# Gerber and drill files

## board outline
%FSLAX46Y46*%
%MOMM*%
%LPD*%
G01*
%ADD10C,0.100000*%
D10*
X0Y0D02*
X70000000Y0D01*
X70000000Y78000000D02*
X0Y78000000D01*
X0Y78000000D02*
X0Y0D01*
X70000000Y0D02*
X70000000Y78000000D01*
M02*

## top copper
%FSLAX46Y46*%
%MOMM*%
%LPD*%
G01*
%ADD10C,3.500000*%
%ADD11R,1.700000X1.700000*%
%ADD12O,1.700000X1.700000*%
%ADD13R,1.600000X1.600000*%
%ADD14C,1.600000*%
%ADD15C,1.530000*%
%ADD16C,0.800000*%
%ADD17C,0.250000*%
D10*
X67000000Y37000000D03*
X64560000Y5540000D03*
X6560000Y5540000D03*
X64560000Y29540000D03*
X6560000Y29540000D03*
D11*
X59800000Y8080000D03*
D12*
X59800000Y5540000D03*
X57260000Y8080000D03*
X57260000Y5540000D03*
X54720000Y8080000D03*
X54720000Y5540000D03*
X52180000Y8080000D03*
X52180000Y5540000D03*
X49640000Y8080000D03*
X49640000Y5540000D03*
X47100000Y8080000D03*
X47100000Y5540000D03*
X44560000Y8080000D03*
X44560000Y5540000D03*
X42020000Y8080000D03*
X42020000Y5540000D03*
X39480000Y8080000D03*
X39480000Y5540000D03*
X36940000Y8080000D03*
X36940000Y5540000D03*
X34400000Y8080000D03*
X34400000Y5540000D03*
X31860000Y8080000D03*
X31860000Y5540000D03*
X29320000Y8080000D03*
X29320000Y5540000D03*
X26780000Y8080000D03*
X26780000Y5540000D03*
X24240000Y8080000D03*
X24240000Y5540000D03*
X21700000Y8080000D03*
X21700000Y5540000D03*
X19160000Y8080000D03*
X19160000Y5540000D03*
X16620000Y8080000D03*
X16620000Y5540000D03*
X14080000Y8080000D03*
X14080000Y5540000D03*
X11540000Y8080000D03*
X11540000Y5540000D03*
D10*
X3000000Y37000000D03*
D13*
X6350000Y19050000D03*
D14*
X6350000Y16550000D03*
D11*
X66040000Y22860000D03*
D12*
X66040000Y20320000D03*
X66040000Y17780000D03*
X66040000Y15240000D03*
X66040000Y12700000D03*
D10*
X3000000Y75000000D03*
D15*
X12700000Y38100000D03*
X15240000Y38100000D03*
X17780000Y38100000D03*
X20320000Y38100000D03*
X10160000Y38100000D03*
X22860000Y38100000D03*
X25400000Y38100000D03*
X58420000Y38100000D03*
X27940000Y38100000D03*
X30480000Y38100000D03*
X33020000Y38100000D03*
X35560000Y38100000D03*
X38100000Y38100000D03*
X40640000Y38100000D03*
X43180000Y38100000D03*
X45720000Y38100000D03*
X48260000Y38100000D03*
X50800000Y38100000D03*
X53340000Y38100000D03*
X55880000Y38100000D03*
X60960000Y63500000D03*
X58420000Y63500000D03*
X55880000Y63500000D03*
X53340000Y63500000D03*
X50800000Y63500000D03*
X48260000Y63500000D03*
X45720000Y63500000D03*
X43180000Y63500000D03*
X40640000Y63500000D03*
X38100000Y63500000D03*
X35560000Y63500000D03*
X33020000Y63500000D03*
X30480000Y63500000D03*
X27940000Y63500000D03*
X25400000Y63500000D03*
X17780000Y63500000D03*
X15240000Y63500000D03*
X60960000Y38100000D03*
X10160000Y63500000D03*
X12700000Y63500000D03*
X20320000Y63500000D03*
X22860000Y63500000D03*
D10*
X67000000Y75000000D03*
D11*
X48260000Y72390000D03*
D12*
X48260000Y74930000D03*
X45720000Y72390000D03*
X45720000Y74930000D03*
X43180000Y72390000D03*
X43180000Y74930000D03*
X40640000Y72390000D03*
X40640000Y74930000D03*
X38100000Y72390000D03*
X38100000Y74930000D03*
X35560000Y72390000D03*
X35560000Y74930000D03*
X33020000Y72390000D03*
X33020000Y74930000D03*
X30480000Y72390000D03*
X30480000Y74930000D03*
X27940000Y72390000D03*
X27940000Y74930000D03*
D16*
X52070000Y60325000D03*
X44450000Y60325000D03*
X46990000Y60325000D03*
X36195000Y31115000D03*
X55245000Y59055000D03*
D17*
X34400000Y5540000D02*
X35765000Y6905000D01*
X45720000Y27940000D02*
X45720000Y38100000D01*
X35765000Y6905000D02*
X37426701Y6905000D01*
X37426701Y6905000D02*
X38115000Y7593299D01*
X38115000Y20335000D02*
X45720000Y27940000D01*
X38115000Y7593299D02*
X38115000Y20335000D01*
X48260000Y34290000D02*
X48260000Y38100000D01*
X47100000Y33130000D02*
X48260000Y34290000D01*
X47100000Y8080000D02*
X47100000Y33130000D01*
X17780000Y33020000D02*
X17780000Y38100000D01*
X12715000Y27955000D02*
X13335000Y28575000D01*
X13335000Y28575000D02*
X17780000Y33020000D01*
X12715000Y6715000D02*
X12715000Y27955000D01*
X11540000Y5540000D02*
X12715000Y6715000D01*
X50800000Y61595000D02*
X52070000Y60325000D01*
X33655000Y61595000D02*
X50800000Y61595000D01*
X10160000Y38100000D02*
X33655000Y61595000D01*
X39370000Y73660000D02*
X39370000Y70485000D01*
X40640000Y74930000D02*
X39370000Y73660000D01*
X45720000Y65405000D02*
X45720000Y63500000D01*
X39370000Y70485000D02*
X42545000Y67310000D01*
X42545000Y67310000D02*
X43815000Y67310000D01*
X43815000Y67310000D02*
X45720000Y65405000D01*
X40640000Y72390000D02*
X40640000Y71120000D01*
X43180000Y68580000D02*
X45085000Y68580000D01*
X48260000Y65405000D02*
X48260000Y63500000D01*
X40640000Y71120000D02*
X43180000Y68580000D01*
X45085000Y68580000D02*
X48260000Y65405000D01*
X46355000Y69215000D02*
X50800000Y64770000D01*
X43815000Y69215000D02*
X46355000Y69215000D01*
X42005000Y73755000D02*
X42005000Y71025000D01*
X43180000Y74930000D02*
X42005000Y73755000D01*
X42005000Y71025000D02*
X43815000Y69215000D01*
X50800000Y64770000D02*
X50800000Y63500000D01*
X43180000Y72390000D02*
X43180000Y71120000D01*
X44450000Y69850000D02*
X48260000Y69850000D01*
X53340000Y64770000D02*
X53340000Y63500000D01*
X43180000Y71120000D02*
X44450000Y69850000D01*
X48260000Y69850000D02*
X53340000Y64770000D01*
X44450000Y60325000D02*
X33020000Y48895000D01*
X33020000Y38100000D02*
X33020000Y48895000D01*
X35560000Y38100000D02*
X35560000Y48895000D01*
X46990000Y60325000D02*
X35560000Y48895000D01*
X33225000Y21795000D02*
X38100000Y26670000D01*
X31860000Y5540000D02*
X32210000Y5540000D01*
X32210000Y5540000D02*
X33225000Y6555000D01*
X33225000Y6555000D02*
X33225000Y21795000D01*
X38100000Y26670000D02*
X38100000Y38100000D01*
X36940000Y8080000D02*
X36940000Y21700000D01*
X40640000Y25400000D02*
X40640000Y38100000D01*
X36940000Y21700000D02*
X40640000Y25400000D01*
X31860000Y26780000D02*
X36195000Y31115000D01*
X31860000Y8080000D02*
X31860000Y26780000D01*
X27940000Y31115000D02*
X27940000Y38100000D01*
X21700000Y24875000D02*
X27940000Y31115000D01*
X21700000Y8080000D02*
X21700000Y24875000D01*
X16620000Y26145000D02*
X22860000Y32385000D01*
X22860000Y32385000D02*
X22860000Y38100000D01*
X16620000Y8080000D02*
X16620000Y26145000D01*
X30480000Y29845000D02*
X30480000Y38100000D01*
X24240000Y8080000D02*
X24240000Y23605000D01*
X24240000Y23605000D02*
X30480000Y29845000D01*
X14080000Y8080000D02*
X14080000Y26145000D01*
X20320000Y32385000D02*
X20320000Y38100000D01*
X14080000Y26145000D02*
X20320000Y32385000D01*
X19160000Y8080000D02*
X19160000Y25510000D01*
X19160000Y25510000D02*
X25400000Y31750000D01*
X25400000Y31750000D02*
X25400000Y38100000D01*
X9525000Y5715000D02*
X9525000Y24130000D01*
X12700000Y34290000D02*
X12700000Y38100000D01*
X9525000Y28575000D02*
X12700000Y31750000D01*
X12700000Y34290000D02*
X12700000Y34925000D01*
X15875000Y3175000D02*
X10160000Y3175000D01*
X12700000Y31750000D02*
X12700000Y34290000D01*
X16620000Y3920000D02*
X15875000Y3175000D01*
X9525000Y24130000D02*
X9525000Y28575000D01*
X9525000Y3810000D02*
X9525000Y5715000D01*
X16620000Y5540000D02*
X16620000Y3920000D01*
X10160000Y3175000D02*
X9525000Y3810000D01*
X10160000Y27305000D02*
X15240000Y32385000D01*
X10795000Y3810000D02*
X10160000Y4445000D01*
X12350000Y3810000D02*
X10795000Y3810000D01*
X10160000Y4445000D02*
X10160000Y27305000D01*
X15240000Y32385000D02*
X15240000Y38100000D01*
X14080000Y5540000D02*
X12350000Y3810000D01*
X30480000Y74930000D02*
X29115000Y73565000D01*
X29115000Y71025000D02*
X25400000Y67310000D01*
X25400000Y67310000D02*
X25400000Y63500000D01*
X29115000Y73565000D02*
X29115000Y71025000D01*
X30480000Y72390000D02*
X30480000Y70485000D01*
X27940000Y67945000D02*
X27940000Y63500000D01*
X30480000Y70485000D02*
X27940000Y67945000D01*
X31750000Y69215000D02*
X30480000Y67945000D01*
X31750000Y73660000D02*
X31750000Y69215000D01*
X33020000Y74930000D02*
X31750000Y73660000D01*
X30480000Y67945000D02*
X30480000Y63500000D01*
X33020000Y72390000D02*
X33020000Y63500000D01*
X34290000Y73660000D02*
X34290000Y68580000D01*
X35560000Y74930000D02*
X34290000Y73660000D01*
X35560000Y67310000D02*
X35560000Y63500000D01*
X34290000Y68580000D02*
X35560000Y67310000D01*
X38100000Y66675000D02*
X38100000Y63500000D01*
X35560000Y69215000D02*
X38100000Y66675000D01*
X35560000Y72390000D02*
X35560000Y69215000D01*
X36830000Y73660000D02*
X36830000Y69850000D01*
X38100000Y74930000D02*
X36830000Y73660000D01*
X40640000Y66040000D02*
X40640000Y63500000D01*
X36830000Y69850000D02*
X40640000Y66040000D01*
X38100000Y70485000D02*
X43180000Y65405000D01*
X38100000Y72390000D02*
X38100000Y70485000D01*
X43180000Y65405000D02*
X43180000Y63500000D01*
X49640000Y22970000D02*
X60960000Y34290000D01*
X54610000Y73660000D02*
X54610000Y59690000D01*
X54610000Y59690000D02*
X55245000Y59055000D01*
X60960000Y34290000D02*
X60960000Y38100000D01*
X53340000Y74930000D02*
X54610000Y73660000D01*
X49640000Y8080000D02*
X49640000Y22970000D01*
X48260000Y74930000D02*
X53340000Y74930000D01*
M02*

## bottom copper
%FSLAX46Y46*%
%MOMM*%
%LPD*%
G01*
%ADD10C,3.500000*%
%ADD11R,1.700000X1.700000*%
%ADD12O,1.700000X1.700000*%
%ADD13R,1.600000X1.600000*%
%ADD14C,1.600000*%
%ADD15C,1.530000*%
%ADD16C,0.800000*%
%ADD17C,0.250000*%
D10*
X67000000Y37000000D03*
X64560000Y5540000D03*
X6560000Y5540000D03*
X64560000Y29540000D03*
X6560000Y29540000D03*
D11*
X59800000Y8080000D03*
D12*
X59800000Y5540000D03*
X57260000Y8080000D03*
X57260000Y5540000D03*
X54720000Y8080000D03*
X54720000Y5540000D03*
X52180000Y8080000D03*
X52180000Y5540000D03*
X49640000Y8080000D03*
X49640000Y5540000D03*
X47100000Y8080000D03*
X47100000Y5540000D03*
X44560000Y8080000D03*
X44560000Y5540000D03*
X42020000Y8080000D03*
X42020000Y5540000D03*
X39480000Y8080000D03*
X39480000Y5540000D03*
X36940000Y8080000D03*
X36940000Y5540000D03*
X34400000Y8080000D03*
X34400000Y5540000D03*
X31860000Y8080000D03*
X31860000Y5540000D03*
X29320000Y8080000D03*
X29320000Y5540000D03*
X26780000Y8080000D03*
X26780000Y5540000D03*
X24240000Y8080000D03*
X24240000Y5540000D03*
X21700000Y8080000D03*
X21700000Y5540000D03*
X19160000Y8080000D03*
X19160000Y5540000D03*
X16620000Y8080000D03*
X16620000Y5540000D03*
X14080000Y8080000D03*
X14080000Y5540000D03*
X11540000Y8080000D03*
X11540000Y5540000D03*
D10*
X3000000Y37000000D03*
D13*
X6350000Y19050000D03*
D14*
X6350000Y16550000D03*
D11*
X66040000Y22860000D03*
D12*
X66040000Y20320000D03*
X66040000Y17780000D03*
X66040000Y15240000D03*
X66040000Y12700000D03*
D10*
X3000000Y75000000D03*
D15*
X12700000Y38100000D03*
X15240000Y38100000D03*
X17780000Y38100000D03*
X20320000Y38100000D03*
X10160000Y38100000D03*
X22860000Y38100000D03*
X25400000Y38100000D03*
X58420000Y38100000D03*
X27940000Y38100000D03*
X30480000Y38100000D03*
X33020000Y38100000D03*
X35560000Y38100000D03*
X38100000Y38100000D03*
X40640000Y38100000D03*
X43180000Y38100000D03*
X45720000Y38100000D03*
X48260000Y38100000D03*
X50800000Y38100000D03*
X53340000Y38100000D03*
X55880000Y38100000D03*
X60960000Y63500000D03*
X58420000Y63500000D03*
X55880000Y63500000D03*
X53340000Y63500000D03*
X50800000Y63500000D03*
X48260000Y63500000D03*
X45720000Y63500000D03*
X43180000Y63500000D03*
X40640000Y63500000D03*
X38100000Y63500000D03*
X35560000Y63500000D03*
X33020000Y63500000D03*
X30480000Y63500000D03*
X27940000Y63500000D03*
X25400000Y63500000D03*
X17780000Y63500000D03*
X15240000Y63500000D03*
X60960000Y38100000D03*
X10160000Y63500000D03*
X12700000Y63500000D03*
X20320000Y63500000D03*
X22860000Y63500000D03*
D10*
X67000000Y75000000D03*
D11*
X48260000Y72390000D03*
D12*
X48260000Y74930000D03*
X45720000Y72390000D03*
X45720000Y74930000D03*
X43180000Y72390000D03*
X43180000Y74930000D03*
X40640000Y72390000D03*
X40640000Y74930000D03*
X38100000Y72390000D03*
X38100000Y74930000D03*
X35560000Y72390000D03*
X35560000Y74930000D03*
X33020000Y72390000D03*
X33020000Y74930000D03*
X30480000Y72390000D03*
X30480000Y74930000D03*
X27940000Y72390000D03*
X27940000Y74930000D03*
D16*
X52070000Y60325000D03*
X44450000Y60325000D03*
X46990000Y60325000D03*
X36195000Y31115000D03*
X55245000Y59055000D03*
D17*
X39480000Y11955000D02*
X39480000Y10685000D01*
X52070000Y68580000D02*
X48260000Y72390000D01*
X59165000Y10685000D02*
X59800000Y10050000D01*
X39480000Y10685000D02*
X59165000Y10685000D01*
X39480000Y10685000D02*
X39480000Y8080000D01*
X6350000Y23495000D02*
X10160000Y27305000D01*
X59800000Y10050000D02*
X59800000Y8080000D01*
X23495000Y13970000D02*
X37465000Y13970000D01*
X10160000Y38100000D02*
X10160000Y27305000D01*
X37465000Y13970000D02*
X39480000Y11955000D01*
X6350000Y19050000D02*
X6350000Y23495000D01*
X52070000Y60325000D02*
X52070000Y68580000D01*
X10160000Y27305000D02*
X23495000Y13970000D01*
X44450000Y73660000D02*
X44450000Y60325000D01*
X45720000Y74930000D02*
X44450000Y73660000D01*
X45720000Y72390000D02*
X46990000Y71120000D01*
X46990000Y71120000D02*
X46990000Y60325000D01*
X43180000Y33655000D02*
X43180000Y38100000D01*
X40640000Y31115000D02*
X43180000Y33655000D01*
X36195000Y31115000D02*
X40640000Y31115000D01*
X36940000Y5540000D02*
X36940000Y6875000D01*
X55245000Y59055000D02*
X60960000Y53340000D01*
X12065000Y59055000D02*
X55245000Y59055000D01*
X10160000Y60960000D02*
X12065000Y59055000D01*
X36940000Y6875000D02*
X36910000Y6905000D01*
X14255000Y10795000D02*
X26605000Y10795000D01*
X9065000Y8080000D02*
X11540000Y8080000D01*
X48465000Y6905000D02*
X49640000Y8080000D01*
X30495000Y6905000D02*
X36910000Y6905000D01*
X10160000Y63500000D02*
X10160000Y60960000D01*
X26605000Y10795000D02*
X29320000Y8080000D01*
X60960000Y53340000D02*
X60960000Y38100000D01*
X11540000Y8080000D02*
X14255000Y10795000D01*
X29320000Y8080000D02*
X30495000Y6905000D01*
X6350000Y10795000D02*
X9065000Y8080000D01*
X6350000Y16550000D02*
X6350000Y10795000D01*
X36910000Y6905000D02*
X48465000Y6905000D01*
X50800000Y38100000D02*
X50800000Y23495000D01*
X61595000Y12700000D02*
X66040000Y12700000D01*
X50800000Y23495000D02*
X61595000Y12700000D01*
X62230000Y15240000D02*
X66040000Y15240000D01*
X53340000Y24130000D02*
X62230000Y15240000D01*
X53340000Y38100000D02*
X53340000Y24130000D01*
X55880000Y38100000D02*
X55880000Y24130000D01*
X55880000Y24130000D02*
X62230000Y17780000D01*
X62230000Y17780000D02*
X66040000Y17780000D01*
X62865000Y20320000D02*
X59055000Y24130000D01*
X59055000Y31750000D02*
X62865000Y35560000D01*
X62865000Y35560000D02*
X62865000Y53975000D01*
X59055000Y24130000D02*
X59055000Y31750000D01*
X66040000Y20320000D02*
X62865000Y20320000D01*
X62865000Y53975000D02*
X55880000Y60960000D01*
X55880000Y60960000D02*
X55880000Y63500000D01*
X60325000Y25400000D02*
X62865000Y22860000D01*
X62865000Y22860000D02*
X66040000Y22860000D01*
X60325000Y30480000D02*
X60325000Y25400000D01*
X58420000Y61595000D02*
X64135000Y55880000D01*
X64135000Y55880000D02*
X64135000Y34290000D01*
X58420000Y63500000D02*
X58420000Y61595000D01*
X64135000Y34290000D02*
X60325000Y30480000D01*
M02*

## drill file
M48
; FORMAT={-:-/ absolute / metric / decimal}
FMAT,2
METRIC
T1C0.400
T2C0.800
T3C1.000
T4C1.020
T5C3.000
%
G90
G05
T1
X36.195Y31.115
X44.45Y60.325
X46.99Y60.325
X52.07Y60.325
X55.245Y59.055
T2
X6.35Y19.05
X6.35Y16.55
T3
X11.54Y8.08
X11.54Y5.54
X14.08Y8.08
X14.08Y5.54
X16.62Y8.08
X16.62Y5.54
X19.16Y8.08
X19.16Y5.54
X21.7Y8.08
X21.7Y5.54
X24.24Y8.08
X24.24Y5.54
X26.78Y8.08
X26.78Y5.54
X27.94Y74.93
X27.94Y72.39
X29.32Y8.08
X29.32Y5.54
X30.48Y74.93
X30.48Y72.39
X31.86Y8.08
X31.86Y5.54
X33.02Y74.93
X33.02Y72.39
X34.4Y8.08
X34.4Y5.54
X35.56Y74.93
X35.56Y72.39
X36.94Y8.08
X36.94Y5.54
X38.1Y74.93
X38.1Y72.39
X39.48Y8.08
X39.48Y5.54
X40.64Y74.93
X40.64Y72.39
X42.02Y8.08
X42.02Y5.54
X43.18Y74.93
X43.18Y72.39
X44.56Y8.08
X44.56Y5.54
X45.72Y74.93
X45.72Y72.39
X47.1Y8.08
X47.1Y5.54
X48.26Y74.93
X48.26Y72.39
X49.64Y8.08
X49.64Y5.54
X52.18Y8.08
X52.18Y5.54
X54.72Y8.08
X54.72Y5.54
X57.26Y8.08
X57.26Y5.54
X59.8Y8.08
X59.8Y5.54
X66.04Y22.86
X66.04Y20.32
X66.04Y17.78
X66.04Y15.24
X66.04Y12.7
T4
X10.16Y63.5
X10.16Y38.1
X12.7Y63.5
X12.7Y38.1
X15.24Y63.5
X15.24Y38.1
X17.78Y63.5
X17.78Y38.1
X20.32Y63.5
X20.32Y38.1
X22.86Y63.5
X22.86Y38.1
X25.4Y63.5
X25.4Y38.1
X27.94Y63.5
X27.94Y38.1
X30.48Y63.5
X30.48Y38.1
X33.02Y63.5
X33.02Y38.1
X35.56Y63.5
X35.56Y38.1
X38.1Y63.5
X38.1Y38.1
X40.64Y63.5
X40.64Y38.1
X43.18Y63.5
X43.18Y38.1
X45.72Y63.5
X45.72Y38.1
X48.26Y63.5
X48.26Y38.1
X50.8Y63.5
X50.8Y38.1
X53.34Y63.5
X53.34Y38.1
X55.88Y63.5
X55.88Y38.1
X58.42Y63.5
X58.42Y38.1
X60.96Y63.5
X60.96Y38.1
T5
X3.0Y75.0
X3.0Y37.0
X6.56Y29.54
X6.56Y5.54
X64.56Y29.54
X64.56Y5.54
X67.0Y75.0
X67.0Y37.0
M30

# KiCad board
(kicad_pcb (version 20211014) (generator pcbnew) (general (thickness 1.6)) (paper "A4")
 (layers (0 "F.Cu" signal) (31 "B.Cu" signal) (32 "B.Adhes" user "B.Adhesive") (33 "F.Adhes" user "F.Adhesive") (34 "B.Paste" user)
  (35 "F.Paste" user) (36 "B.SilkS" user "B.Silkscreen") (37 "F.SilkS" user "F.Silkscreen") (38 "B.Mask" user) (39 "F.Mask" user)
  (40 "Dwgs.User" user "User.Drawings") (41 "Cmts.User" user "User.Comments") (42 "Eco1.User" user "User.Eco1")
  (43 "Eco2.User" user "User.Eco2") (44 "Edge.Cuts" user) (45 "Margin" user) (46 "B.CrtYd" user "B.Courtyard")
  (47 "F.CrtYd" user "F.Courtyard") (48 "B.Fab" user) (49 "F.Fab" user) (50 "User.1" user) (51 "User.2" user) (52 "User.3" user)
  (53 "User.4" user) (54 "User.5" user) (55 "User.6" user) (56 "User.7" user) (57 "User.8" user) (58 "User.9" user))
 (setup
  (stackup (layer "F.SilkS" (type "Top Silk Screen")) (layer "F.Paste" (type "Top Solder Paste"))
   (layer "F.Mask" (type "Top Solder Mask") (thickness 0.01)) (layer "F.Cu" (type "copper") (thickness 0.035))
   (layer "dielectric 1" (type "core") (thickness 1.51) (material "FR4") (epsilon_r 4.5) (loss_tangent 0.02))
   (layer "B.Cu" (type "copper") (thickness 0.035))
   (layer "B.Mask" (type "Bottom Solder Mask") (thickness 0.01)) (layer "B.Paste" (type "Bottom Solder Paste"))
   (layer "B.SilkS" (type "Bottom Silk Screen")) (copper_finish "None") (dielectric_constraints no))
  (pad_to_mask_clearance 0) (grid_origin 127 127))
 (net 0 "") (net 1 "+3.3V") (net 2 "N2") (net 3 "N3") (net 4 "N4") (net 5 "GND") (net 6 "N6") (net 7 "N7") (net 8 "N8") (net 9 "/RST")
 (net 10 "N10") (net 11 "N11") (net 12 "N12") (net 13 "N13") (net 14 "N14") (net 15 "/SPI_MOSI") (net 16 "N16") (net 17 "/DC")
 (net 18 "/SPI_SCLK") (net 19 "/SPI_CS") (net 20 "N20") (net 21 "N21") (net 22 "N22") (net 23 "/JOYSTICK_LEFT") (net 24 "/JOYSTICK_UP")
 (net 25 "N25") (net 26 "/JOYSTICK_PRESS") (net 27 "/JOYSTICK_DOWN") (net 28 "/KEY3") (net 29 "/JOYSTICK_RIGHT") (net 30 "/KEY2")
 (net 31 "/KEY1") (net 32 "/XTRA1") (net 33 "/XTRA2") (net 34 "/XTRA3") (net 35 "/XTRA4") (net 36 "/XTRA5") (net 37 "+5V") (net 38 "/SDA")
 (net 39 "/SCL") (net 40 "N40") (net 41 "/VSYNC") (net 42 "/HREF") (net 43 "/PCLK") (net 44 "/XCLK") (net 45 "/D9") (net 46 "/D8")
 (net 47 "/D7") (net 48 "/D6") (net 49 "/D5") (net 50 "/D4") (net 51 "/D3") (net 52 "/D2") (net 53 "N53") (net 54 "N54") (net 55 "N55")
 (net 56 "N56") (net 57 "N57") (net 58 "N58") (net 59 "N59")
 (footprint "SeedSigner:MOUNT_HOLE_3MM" (layer "F.Cu") (at 67 -37)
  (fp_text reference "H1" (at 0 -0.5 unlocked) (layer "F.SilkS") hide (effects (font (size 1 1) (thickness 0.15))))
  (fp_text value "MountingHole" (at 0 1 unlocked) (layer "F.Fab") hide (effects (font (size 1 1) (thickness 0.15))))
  (pad "" np_thru_hole circle (at 0 0) (size 3.5 3.5) (drill 3) (layers F&B.Cu *.Mask)))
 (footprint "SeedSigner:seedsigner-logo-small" (layer "F.Cu") (at 15.24 -73.025)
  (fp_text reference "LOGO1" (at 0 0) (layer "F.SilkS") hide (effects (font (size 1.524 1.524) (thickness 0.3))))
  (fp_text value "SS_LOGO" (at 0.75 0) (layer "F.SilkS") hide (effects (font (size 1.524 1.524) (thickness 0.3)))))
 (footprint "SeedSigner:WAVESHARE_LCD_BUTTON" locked (layer "F.Cu") (at 35.56 -17.54 180)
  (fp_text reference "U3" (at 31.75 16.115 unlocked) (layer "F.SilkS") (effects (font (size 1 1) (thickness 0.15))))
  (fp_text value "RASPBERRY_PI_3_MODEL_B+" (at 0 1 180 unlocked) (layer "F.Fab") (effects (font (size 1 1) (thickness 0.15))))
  (pad "" np_thru_hole circle locked (at -29 -12 180) (size 3.5 3.5) (drill 3) (layers F&B.Cu *.Mask))
  (pad "" np_thru_hole circle locked (at 29 -12 180) (size 3.5 3.5) (drill 3) (layers F&B.Cu *.Mask))
  (pad "" np_thru_hole circle locked (at -29 12 180) (size 3.5 3.5) (drill 3) (layers F&B.Cu *.Mask))
  (pad "" np_thru_hole circle locked (at 29 12 180) (size 3.5 3.5) (drill 3) (layers F&B.Cu *.Mask))
  (pad "1" thru_hole rect locked (at -24.24 -9.46 270) (size 1.7 1.7) (drill 1) (layers *.Cu *.Mask) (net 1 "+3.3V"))
  (pad "2" thru_hole oval locked (at -24.24 -12 270) (size 1.7 1.7) (drill 1) (layers *.Cu *.Mask) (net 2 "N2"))
  (pad "3" thru_hole oval locked (at -21.7 -9.46 270) (size 1.7 1.7) (drill 1) (layers *.Cu *.Mask) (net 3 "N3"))
  (pad "4" thru_hole oval locked (at -21.7 -12 270) (size 1.7 1.7) (drill 1) (layers *.Cu *.Mask) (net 2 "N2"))
  (pad "5" thru_hole oval locked (at -19.16 -9.46 270) (size 1.7 1.7) (drill 1) (layers *.Cu *.Mask) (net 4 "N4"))
  (pad "6" thru_hole oval locked (at -19.16 -12 270) (size 1.7 1.7) (drill 1) (layers *.Cu *.Mask) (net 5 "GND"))
  (pad "7" thru_hole oval locked (at -16.62 -9.46 270) (size 1.7 1.7) (drill 1) (layers *.Cu *.Mask) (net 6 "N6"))
  (pad "8" thru_hole oval locked (at -16.62 -12 270) (size 1.7 1.7) (drill 1) (layers *.Cu *.Mask) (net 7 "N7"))
  (pad "9" thru_hole oval locked (at -14.08 -9.46 270) (size 1.7 1.7) (drill 1) (layers *.Cu *.Mask) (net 5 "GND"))
  (pad "10" thru_hole oval locked (at -14.08 -12 270) (size 1.7 1.7) (drill 1) (layers *.Cu *.Mask) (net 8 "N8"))
  (pad "11" thru_hole oval locked (at -11.54 -9.46 270) (size 1.7 1.7) (drill 1) (layers *.Cu *.Mask) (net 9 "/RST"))
  (pad "12" thru_hole oval locked (at -11.54 -12 270) (size 1.7 1.7) (drill 1) (layers *.Cu *.Mask) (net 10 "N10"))
  (pad "13" thru_hole oval locked (at -9 -9.46 270) (size 1.7 1.7) (drill 1) (layers *.Cu *.Mask) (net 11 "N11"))
  (pad "14" thru_hole oval locked (at -9 -12 270) (size 1.7 1.7) (drill 1) (layers *.Cu *.Mask) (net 5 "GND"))
  (pad "15" thru_hole oval locked (at -6.46 -9.46 270) (size 1.7 1.7) (drill 1) (layers *.Cu *.Mask) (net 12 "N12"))
  (pad "16" thru_hole oval locked (at -6.46 -12 270) (size 1.7 1.7) (drill 1) (layers *.Cu *.Mask) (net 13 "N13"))
  (pad "17" thru_hole oval locked (at -3.92 -9.46 270) (size 1.7 1.7) (drill 1) (layers *.Cu *.Mask) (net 1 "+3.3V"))
  (pad "18" thru_hole oval locked (at -3.92 -12 270) (size 1.7 1.7) (drill 1) (layers *.Cu *.Mask) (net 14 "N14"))
  (pad "19" thru_hole oval locked (at -1.38 -9.46 270) (size 1.7 1.7) (drill 1) (layers *.Cu *.Mask) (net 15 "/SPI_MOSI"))
  (pad "20" thru_hole oval locked (at -1.38 -12 90) (size 1.7 1.7) (drill 1) (layers *.Cu *.Mask) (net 5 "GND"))
  (pad "21" thru_hole oval locked (at 1.16 -9.46 270) (size 1.7 1.7) (drill 1) (layers *.Cu *.Mask) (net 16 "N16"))
  (pad "22" thru_hole oval locked (at 1.16 -12 270) (size 1.7 1.7) (drill 1) (layers *.Cu *.Mask) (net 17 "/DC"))
  (pad "23" thru_hole oval locked (at 3.7 -9.46 270) (size 1.7 1.7) (drill 1) (layers *.Cu *.Mask) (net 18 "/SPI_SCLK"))
  (pad "24" thru_hole oval locked (at 3.7 -12 270) (size 1.7 1.7) (drill 1) (layers *.Cu *.Mask) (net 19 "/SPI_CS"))
  (pad "25" thru_hole oval locked (at 6.24 -9.46 270) (size 1.7 1.7) (drill 1) (layers *.Cu *.Mask) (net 5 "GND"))
  (pad "26" thru_hole oval locked (at 6.24 -12 270) (size 1.7 1.7) (drill 1) (layers *.Cu *.Mask) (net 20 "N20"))
  (pad "27" thru_hole oval locked (at 8.78 -9.46 270) (size 1.7 1.7) (drill 1) (layers *.Cu *.Mask) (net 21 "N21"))
  (pad "28" thru_hole oval locked (at 8.78 -12 270) (size 1.7 1.7) (drill 1) (layers *.Cu *.Mask) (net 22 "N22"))
  (pad "29" thru_hole oval locked (at 11.32 -9.46 270) (size 1.7 1.7) (drill 1) (layers *.Cu *.Mask) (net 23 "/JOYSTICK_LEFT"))
  (pad "30" thru_hole oval locked (at 11.32 -12 270) (size 1.7 1.7) (drill 1) (layers *.Cu *.Mask) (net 5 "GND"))
  (pad "31" thru_hole oval locked (at 13.86 -9.46 270) (size 1.7 1.7) (drill 1) (layers *.Cu *.Mask) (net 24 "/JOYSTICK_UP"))
  (pad "32" thru_hole oval locked (at 13.86 -12 270) (size 1.7 1.7) (drill 1) (layers *.Cu *.Mask) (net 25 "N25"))
  (pad "33" thru_hole oval locked (at 16.4 -9.46 270) (size 1.7 1.7) (drill 1) (layers *.Cu *.Mask) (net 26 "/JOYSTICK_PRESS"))
  (pad "34" thru_hole oval locked (at 16.4 -12 270) (size 1.7 1.7) (drill 1) (layers *.Cu *.Mask) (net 5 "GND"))
  (pad "35" thru_hole oval locked (at 18.94 -9.46 270) (size 1.7 1.7) (drill 1) (layers *.Cu *.Mask) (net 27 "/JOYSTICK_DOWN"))
  (pad "36" thru_hole oval locked (at 18.94 -12 270) (size 1.7 1.7) (drill 1) (layers *.Cu *.Mask) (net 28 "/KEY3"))
  (pad "37" thru_hole oval locked (at 21.48 -9.46 270) (size 1.7 1.7) (drill 1) (layers *.Cu *.Mask) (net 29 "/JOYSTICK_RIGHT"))
  (pad "38" thru_hole oval locked (at 21.48 -12 270) (size 1.7 1.7) (drill 1) (layers *.Cu *.Mask) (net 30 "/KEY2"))
  (pad "39" thru_hole oval locked (at 24.02 -9.46 270) (size 1.7 1.7) (drill 1) (layers *.Cu *.Mask) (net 5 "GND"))
  (pad "40" thru_hole oval locked (at 24.02 -12 270) (size 1.7 1.7) (drill 1) (layers *.Cu *.Mask) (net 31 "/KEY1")))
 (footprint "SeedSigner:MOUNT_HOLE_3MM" (layer "F.Cu") (at 3 -37)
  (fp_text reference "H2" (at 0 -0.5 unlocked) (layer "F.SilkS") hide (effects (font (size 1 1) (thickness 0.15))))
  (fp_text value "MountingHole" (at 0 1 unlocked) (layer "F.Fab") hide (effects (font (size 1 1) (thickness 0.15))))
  (pad "" np_thru_hole circle (at 0 0) (size 3.5 3.5) (drill 3) (layers F&B.Cu *.Mask)))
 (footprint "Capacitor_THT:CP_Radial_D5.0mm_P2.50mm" (layer "F.Cu") (at 6.35 -19.05 -90)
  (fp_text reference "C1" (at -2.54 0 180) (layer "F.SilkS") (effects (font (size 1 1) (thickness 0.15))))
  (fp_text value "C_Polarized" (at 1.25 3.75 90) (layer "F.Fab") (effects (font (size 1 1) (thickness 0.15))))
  (pad "1" thru_hole rect (at 0 0 270) (size 1.6 1.6) (drill 0.8) (layers *.Cu *.Mask) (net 1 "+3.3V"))
  (pad "2" thru_hole circle (at 2.5 0 270) (size 1.6 1.6) (drill 0.8) (layers *.Cu *.Mask) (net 5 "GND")))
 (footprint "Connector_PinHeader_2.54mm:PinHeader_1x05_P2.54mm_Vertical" (layer "F.Cu") (at 66.04 -22.86)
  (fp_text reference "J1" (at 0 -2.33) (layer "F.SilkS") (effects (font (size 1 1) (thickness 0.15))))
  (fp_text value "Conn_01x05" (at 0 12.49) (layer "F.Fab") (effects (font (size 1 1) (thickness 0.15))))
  (pad "1" thru_hole rect (at 0 0) (size 1.7 1.7) (drill 1) (layers *.Cu *.Mask) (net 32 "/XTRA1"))
  (pad "2" thru_hole oval (at 0 2.54) (size 1.7 1.7) (drill 1) (layers *.Cu *.Mask) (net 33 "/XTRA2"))
  (pad "3" thru_hole oval (at 0 5.08) (size 1.7 1.7) (drill 1) (layers *.Cu *.Mask) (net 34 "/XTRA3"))
  (pad "4" thru_hole oval (at 0 7.62) (size 1.7 1.7) (drill 1) (layers *.Cu *.Mask) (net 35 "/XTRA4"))
  (pad "5" thru_hole oval (at 0 10.16) (size 1.7 1.7) (drill 1) (layers *.Cu *.Mask) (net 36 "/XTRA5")))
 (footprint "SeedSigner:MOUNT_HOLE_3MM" (layer "F.Cu") (at 3 -75)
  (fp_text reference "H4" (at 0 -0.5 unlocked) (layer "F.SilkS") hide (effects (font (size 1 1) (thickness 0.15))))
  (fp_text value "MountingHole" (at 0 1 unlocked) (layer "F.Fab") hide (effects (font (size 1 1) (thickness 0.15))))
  (pad "" np_thru_hole circle (at 0 0) (size 3.5 3.5) (drill 3) (layers F&B.Cu *.Mask)))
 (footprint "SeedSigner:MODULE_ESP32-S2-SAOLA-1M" (layer "F.Cu") (at 35.56 -50.8 90)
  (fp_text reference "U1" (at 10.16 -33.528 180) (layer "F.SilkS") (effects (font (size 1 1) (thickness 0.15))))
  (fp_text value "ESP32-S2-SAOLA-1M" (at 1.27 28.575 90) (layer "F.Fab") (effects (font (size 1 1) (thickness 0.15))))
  (pad "0" thru_hole circle (at -12.7 -22.86 90) (size 1.53 1.53) (drill 1.02) (layers *.Cu *.Mask) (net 28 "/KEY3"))
  (pad "1" thru_hole circle (at -12.7 -20.32 90) (size 1.53 1.53) (drill 1.02) (layers *.Cu *.Mask) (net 30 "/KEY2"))
  (pad "2" thru_hole circle (at -12.7 -17.78 90) (size 1.53 1.53) (drill 1.02) (layers *.Cu *.Mask) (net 31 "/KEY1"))
  (pad "3" thru_hole circle (at -12.7 -15.24 90) (size 1.53 1.53) (drill 1.02) (layers *.Cu *.Mask) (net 29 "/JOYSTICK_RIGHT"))
  (pad "3V3" thru_hole circle (at -12.7 -25.4 90) (size 1.53 1.53) (drill 1.02) (layers *.Cu *.Mask) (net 1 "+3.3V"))
  (pad "4" thru_hole circle (at -12.7 -12.7 90) (size 1.53 1.53) (drill 1.02) (layers *.Cu *.Mask) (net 27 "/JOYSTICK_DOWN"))
  (pad "5" thru_hole circle (at -12.7 -10.16 90) (size 1.53 1.53) (drill 1.02) (layers *.Cu *.Mask) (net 26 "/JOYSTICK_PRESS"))
  (pad "5V" thru_hole circle (at -12.7 22.86 90) (size 1.53 1.53) (drill 1.02) (layers *.Cu *.Mask) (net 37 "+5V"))
  (pad "6" thru_hole circle (at -12.7 -7.62 90) (size 1.53 1.53) (drill 1.02) (layers *.Cu *.Mask) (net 24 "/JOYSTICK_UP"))
  (pad "7" thru_hole circle (at -12.7 -5.08 90) (size 1.53 1.53) (drill 1.02) (layers *.Cu *.Mask) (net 23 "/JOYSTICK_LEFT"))
  (pad "8" thru_hole circle (at -12.7 -2.54 90) (size 1.53 1.53) (drill 1.02) (layers *.Cu *.Mask) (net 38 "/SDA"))
  (pad "9" thru_hole circle (at -12.7 0 90) (size 1.53 1.53) (drill 1.02) (layers *.Cu *.Mask) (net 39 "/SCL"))
  (pad "10" thru_hole circle (at -12.7 2.54 90) (size 1.53 1.53) (drill 1.02) (layers *.Cu *.Mask) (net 19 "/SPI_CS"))
  (pad "11" thru_hole circle (at -12.7 5.08 90) (size 1.53 1.53) (drill 1.02) (layers *.Cu *.Mask) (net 15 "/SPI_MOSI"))
  (pad "12" thru_hole circle (at -12.7 7.62 90) (size 1.53 1.53) (drill 1.02) (layers *.Cu *.Mask) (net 18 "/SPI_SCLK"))
  (pad "13" thru_hole circle (at -12.7 10.16 90) (size 1.53 1.53) (drill 1.02) (layers *.Cu *.Mask) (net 17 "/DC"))
  (pad "14" thru_hole circle (at -12.7 12.7 90) (size 1.53 1.53) (drill 1.02) (layers *.Cu *.Mask) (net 9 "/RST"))
  (pad "15" thru_hole circle (at -12.7 15.24 90) (size 1.53 1.53) (drill 1.02) (layers *.Cu *.Mask) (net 36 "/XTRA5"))
  (pad "16" thru_hole circle (at -12.7 17.78 90) (size 1.53 1.53) (drill 1.02) (layers *.Cu *.Mask) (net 35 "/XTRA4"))
  (pad "17" thru_hole circle (at -12.7 20.32 90) (size 1.53 1.53) (drill 1.02) (layers *.Cu *.Mask) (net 34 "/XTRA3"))
  (pad "18" thru_hole circle (at 12.7 25.4 90) (size 1.53 1.53) (drill 1.02) (layers *.Cu *.Mask) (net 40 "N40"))
  (pad "19" thru_hole circle (at 12.7 22.86 90) (size 1.53 1.53) (drill 1.02) (layers *.Cu *.Mask) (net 32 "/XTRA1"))
  (pad "20" thru_hole circle (at 12.7 20.32 90) (size 1.53 1.53) (drill 1.02) (layers *.Cu *.Mask) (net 33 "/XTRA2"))
  (pad "21" thru_hole circle (at 12.7 17.78 90) (size 1.53 1.53) (drill 1.02) (layers *.Cu *.Mask) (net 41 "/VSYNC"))
  (pad "26" thru_hole circle (at 12.7 15.24 90) (size 1.53 1.53) (drill 1.02) (layers *.Cu *.Mask) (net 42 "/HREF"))
  (pad "33" thru_hole circle (at 12.7 12.7 90) (size 1.53 1.53) (drill 1.02) (layers *.Cu *.Mask) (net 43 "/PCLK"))
  (pad "34" thru_hole circle (at 12.7 10.16 90) (size 1.53 1.53) (drill 1.02) (layers *.Cu *.Mask) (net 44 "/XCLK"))
  (pad "35" thru_hole circle (at 12.7 7.62 90) (size 1.53 1.53) (drill 1.02) (layers *.Cu *.Mask) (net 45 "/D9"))
  (pad "36" thru_hole circle (at 12.7 5.08 90) (size 1.53 1.53) (drill 1.02) (layers *.Cu *.Mask) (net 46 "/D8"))
  (pad "37" thru_hole circle (at 12.7 2.54 90) (size 1.53 1.53) (drill 1.02) (layers *.Cu *.Mask) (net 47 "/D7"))
  (pad "38" thru_hole circle (at 12.7 0 90) (size 1.53 1.53) (drill 1.02) (layers *.Cu *.Mask) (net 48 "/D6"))
  (pad "39" thru_hole circle (at 12.7 -2.54 90) (size 1.53 1.53) (drill 1.02) (layers *.Cu *.Mask) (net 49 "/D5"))
  (pad "40" thru_hole circle (at 12.7 -5.08 90) (size 1.53 1.53) (drill 1.02) (layers *.Cu *.Mask) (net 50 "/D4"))
  (pad "41" thru_hole circle (at 12.7 -7.62 90) (size 1.53 1.53) (drill 1.02) (layers *.Cu *.Mask) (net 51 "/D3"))
  (pad "42" thru_hole circle (at 12.7 -10.16 90) (size 1.53 1.53) (drill 1.02) (layers *.Cu *.Mask) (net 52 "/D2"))
  (pad "45" thru_hole circle (at 12.7 -17.78 90) (size 1.53 1.53) (drill 1.02) (layers *.Cu *.Mask) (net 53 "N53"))
  (pad "46" thru_hole circle (at 12.7 -20.32 90) (size 1.53 1.53) (drill 1.02) (layers *.Cu *.Mask) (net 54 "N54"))
  (pad "GND_1" thru_hole circle (at -12.7 25.4 90) (size 1.53 1.53) (drill 1.02) (layers *.Cu *.Mask) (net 5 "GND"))
  (pad "GND_2" thru_hole circle (at 12.7 -25.4 90) (size 1.53 1.53) (drill 1.02) (layers *.Cu *.Mask) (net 5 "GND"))
  (pad "RST" thru_hole circle (at 12.7 -22.86 90) (size 1.53 1.53) (drill 1.02) (layers *.Cu *.Mask) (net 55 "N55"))
  (pad "RX" thru_hole circle (at 12.7 -15.24 90) (size 1.53 1.53) (drill 1.02) (layers *.Cu *.Mask) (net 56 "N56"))
  (pad "TX" thru_hole circle (at 12.7 -12.7 90) (size 1.53 1.53) (drill 1.02) (layers *.Cu *.Mask) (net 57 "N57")))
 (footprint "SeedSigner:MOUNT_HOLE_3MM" (layer "F.Cu") (at 67 -75)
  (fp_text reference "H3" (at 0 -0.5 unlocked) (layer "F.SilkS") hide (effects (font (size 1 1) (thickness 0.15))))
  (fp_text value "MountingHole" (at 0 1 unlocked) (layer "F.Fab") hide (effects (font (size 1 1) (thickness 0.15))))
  (pad "" np_thru_hole circle (at 0 0) (size 3.5 3.5) (drill 3) (layers F&B.Cu *.Mask)))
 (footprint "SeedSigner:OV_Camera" (layer "B.Cu") (at 38.1 -73.66 90)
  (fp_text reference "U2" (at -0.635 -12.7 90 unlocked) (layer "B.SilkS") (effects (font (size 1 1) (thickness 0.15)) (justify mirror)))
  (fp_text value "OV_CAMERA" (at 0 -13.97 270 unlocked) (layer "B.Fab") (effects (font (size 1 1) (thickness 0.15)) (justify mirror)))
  (pad "1" thru_hole rect (at -1.27 10.16 90) (size 1.7 1.7) (drill 1) (layers *.Cu *.Mask) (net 1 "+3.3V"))
  (pad "2" thru_hole oval (at 1.27 10.16 90) (size 1.7 1.7) (drill 1) (layers *.Cu *.Mask) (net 5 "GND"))
  (pad "3" thru_hole oval (at -1.27 7.62 90) (size 1.7 1.7) (drill 1) (layers *.Cu *.Mask) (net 39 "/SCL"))
  (pad "4" thru_hole oval (at 1.27 7.62 90) (size 1.7 1.7) (drill 1) (layers *.Cu *.Mask) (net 38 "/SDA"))
  (pad "5" thru_hole oval (at -1.27 5.08 90) (size 1.7 1.7) (drill 1) (layers *.Cu *.Mask) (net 41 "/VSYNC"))
  (pad "6" thru_hole oval (at 1.27 5.08 90) (size 1.7 1.7) (drill 1) (layers *.Cu *.Mask) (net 42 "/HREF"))
  (pad "7" thru_hole oval (at -1.27 2.54 90) (size 1.7 1.7) (drill 1) (layers *.Cu *.Mask) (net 43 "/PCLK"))
  (pad "8" thru_hole oval (at 1.27 2.54 90) (size 1.7 1.7) (drill 1) (layers *.Cu *.Mask) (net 44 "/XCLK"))
  (pad "9" thru_hole oval (at -1.27 0 90) (size 1.7 1.7) (drill 1) (layers *.Cu *.Mask) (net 45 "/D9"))
  (pad "10" thru_hole oval (at 1.27 0 90) (size 1.7 1.7) (drill 1) (layers *.Cu *.Mask) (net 46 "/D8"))
  (pad "11" thru_hole oval (at -1.27 -2.54 90) (size 1.7 1.7) (drill 1) (layers *.Cu *.Mask) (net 47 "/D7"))
  (pad "12" thru_hole oval (at 1.27 -2.54 90) (size 1.7 1.7) (drill 1) (layers *.Cu *.Mask) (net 48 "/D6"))
  (pad "13" thru_hole oval (at -1.27 -5.08 90) (size 1.7 1.7) (drill 1) (layers *.Cu *.Mask) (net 49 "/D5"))
  (pad "14" thru_hole oval (at 1.27 -5.08 90) (size 1.7 1.7) (drill 1) (layers *.Cu *.Mask) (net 50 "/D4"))
  (pad "15" thru_hole oval (at -1.27 -7.62 90) (size 1.7 1.7) (drill 1) (layers *.Cu *.Mask) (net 51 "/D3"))
  (pad "16" thru_hole oval (at 1.27 -7.62 90) (size 1.7 1.7) (drill 1) (layers *.Cu *.Mask) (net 52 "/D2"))
  (pad "17" thru_hole oval (at -1.27 -10.16 90) (size 1.7 1.7) (drill 1) (layers *.Cu *.Mask) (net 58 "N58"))
  (pad "18" thru_hole oval (at 1.27 -10.16 90) (size 1.7 1.7) (drill 1) (layers *.Cu *.Mask) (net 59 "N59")))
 (gr_line (start 0 0) (end 70 0) (layer "Edge.Cuts") (width 0.1))
 (gr_line (start 70 -78) (end 0 -78) (layer "Edge.Cuts") (width 0.1))
 (gr_line (start 0 -78) (end 0 0) (layer "Edge.Cuts") (width 0.1))
 (gr_line (start 70 0) (end 70 -78) (layer "Edge.Cuts") (width 0.1))
 (segment (start 34.4 -5.54) (end 35.765 -6.905) (width 0.25) (layer "F.Cu") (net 17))
 (segment (start 45.72 -27.94) (end 45.72 -38.1) (width 0.25) (layer "F.Cu") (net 17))
 (segment (start 35.765 -6.905) (end 37.426701 -6.905) (width 0.25) (layer "F.Cu") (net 17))
 (segment (start 37.426701 -6.905) (end 38.115 -7.593299) (width 0.25) (layer "F.Cu") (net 17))
 (segment (start 38.115 -20.335) (end 45.72 -27.94) (width 0.25) (layer "F.Cu") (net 17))
 (segment (start 38.115 -7.593299) (end 38.115 -20.335) (width 0.25) (layer "F.Cu") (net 17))
 (segment (start 48.26 -34.29) (end 48.26 -38.1) (width 0.25) (layer "F.Cu") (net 9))
 (segment (start 47.1 -33.13) (end 48.26 -34.29) (width 0.25) (layer "F.Cu") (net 9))
 (segment (start 47.1 -8.08) (end 47.1 -33.13) (width 0.25) (layer "F.Cu") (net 9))
 (segment (start 17.78 -33.02) (end 17.78 -38.1) (width 0.25) (layer "F.Cu") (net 31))
 (segment (start 12.715 -27.955) (end 13.335 -28.575) (width 0.25) (layer "F.Cu") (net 31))
 (segment (start 13.335 -28.575) (end 17.78 -33.02) (width 0.25) (layer "F.Cu") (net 31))
 (segment (start 12.715 -6.715) (end 12.715 -27.955) (width 0.25) (layer "F.Cu") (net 31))
 (segment (start 11.54 -5.54) (end 12.715 -6.715) (width 0.25) (layer "F.Cu") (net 31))
 (segment (start 50.8 -61.595) (end 52.07 -60.325) (width 0.25) (layer "F.Cu") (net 1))
 (segment (start 33.655 -61.595) (end 50.8 -61.595) (width 0.25) (layer "F.Cu") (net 1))
 (segment (start 10.16 -38.1) (end 33.655 -61.595) (width 0.25) (layer "F.Cu") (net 1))
 (via (at 52.07 -60.325) (size 0.8) (drill 0.4) (layers "F.Cu" "B.Cu") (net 1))
 (segment (start 39.48 -11.955) (end 39.48 -10.685) (width 0.25) (layer "B.Cu") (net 1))
 (segment (start 52.07 -68.58) (end 48.26 -72.39) (width 0.25) (layer "B.Cu") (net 1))
 (segment (start 59.165 -10.685) (end 59.8 -10.05) (width 0.25) (layer "B.Cu") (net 1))
 (segment (start 39.48 -10.685) (end 59.165 -10.685) (width 0.25) (layer "B.Cu") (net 1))
 (segment (start 39.48 -10.685) (end 39.48 -8.08) (width 0.25) (layer "B.Cu") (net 1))
 (segment (start 6.35 -23.495) (end 10.16 -27.305) (width 0.25) (layer "B.Cu") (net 1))
 (segment (start 59.8 -10.05) (end 59.8 -8.08) (width 0.25) (layer "B.Cu") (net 1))
 (segment (start 23.495 -13.97) (end 37.465 -13.97) (width 0.25) (layer "B.Cu") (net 1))
 (segment (start 10.16 -38.1) (end 10.16 -27.305) (width 0.25) (layer "B.Cu") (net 1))
 (segment (start 37.465 -13.97) (end 39.48 -11.955) (width 0.25) (layer "B.Cu") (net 1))
 (segment (start 6.35 -19.05) (end 6.35 -23.495) (width 0.25) (layer "B.Cu") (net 1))
 (segment (start 52.07 -60.325) (end 52.07 -68.58) (width 0.25) (layer "B.Cu") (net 1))
 (segment (start 10.16 -27.305) (end 23.495 -13.97) (width 0.25) (layer "B.Cu") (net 1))
 (segment (start 39.37 -73.66) (end 39.37 -70.485) (width 0.25) (layer "F.Cu") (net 44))
 (segment (start 40.64 -74.93) (end 39.37 -73.66) (width 0.25) (layer "F.Cu") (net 44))
 (segment (start 45.72 -65.405) (end 45.72 -63.5) (width 0.25) (layer "F.Cu") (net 44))
 (segment (start 39.37 -70.485) (end 42.545 -67.31) (width 0.25) (layer "F.Cu") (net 44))
 (segment (start 42.545 -67.31) (end 43.815 -67.31) (width 0.25) (layer "F.Cu") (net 44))
 (segment (start 43.815 -67.31) (end 45.72 -65.405) (width 0.25) (layer "F.Cu") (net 44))
 (segment (start 40.64 -72.39) (end 40.64 -71.12) (width 0.25) (layer "F.Cu") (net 43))
 (segment (start 43.18 -68.58) (end 45.085 -68.58) (width 0.25) (layer "F.Cu") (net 43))
 (segment (start 48.26 -65.405) (end 48.26 -63.5) (width 0.25) (layer "F.Cu") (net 43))
 (segment (start 40.64 -71.12) (end 43.18 -68.58) (width 0.25) (layer "F.Cu") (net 43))
 (segment (start 45.085 -68.58) (end 48.26 -65.405) (width 0.25) (layer "F.Cu") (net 43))
 (segment (start 46.355 -69.215) (end 50.8 -64.77) (width 0.25) (layer "F.Cu") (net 42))
 (segment (start 43.815 -69.215) (end 46.355 -69.215) (width 0.25) (layer "F.Cu") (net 42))
 (segment (start 42.005 -73.755) (end 42.005 -71.025) (width 0.25) (layer "F.Cu") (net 42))
 (segment (start 43.18 -74.93) (end 42.005 -73.755) (width 0.25) (layer "F.Cu") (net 42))
 (segment (start 42.005 -71.025) (end 43.815 -69.215) (width 0.25) (layer "F.Cu") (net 42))
 (segment (start 50.8 -64.77) (end 50.8 -63.5) (width 0.25) (layer "F.Cu") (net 42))
 (segment (start 43.18 -72.39) (end 43.18 -71.12) (width 0.25) (layer "F.Cu") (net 41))
 (segment (start 44.45 -69.85) (end 48.26 -69.85) (width 0.25) (layer "F.Cu") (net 41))
 (segment (start 53.34 -64.77) (end 53.34 -63.5) (width 0.25) (layer "F.Cu") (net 41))
 (segment (start 43.18 -71.12) (end 44.45 -69.85) (width 0.25) (layer "F.Cu") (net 41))
 (segment (start 48.26 -69.85) (end 53.34 -64.77) (width 0.25) (layer "F.Cu") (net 41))
 (segment (start 44.45 -60.325) (end 33.02 -48.895) (width 0.25) (layer "F.Cu") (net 38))
 (segment (start 33.02 -38.1) (end 33.02 -48.895) (width 0.25) (layer "F.Cu") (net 38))
 (via (at 44.45 -60.325) (size 0.8) (drill 0.4) (layers "F.Cu" "B.Cu") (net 38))
 (segment (start 44.45 -73.66) (end 44.45 -60.325) (width 0.25) (layer "B.Cu") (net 38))
 (segment (start 45.72 -74.93) (end 44.45 -73.66) (width 0.25) (layer "B.Cu") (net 38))
 (segment (start 35.56 -38.1) (end 35.56 -48.895) (width 0.25) (layer "F.Cu") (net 39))
 (segment (start 46.99 -60.325) (end 35.56 -48.895) (width 0.25) (layer "F.Cu") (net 39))
 (via (at 46.99 -60.325) (size 0.8) (drill 0.4) (layers "F.Cu" "B.Cu") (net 39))
 (segment (start 45.72 -72.39) (end 46.99 -71.12) (width 0.25) (layer "B.Cu") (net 39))
 (segment (start 46.99 -71.12) (end 46.99 -60.325) (width 0.25) (layer "B.Cu") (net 39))
 (segment (start 33.225 -21.795) (end 38.1 -26.67) (width 0.25) (layer "F.Cu") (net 19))
 (segment (start 31.86 -5.54) (end 32.21 -5.54) (width 0.25) (layer "F.Cu") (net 19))
 (segment (start 32.21 -5.54) (end 33.225 -6.555) (width 0.25) (layer "F.Cu") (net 19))
 (segment (start 33.225 -6.555) (end 33.225 -21.795) (width 0.25) (layer "F.Cu") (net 19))
 (segment (start 38.1 -26.67) (end 38.1 -38.1) (width 0.25) (layer "F.Cu") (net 19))
 (segment (start 36.94 -8.08) (end 36.94 -21.7) (width 0.25) (layer "F.Cu") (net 15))
 (segment (start 40.64 -25.4) (end 40.64 -38.1) (width 0.25) (layer "F.Cu") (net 15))
 (segment (start 36.94 -21.7) (end 40.64 -25.4) (width 0.25) (layer "F.Cu") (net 15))
 (segment (start 31.86 -26.78) (end 36.195 -31.115) (width 0.25) (layer "F.Cu") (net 18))
 (segment (start 31.86 -8.08) (end 31.86 -26.78) (width 0.25) (layer "F.Cu") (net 18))
 (via (at 36.195 -31.115) (size 0.8) (drill 0.4) (layers "F.Cu" "B.Cu") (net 18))
 (segment (start 43.18 -33.655) (end 43.18 -38.1) (width 0.25) (layer "B.Cu") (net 18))
 (segment (start 40.64 -31.115) (end 43.18 -33.655) (width 0.25) (layer "B.Cu") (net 18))
 (segment (start 36.195 -31.115) (end 40.64 -31.115) (width 0.25) (layer "B.Cu") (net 18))
 (segment (start 27.94 -31.115) (end 27.94 -38.1) (width 0.25) (layer "F.Cu") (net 24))
 (segment (start 21.7 -24.875) (end 27.94 -31.115) (width 0.25) (layer "F.Cu") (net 24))
 (segment (start 21.7 -8.08) (end 21.7 -24.875) (width 0.25) (layer "F.Cu") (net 24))
 (segment (start 16.62 -26.145) (end 22.86 -32.385) (width 0.25) (layer "F.Cu") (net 27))
 (segment (start 22.86 -32.385) (end 22.86 -38.1) (width 0.25) (layer "F.Cu") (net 27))
 (segment (start 16.62 -8.08) (end 16.62 -26.145) (width 0.25) (layer "F.Cu") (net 27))
 (segment (start 30.48 -29.845) (end 30.48 -38.1) (width 0.25) (layer "F.Cu") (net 23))
 (segment (start 24.24 -8.08) (end 24.24 -23.605) (width 0.25) (layer "F.Cu") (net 23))
 (segment (start 24.24 -23.605) (end 30.48 -29.845) (width 0.25) (layer "F.Cu") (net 23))
 (segment (start 14.08 -8.08) (end 14.08 -26.145) (width 0.25) (layer "F.Cu") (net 29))
 (segment (start 20.32 -32.385) (end 20.32 -38.1) (width 0.25) (layer "F.Cu") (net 29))
 (segment (start 14.08 -26.145) (end 20.32 -32.385) (width 0.25) (layer "F.Cu") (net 29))
 (segment (start 19.16 -8.08) (end 19.16 -25.51) (width 0.25) (layer "F.Cu") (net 26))
 (segment (start 19.16 -25.51) (end 25.4 -31.75) (width 0.25) (layer "F.Cu") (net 26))
 (segment (start 25.4 -31.75) (end 25.4 -38.1) (width 0.25) (layer "F.Cu") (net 26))
 (segment (start 9.525 -5.715) (end 9.525 -24.13) (width 0.25) (layer "F.Cu") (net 28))
 (segment (start 12.7 -34.29) (end 12.7 -38.1) (width 0.25) (layer "F.Cu") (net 28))
 (segment (start 9.525 -28.575) (end 12.7 -31.75) (width 0.25) (layer "F.Cu") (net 28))
 (segment (start 12.7 -34.29) (end 12.7 -34.925) (width 0.25) (layer "F.Cu") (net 28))
 (segment (start 15.875 -3.175) (end 10.16 -3.175) (width 0.25) (layer "F.Cu") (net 28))
 (segment (start 12.7 -31.75) (end 12.7 -34.29) (width 0.25) (layer "F.Cu") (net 28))
 (segment (start 16.62 -3.92) (end 15.875 -3.175) (width 0.25) (layer "F.Cu") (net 28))
 (segment (start 9.525 -24.13) (end 9.525 -28.575) (width 0.25) (layer "F.Cu") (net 28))
 (segment (start 9.525 -3.81) (end 9.525 -5.715) (width 0.25) (layer "F.Cu") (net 28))
 (segment (start 16.62 -5.54) (end 16.62 -3.92) (width 0.25) (layer "F.Cu") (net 28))
 (segment (start 10.16 -3.175) (end 9.525 -3.81) (width 0.25) (layer "F.Cu") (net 28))
 (segment (start 10.16 -27.305) (end 15.24 -32.385) (width 0.25) (layer "F.Cu") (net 30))
 (segment (start 10.795 -3.81) (end 10.16 -4.445) (width 0.25) (layer "F.Cu") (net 30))
 (segment (start 12.35 -3.81) (end 10.795 -3.81) (width 0.25) (layer "F.Cu") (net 30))
 (segment (start 10.16 -4.445) (end 10.16 -27.305) (width 0.25) (layer "F.Cu") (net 30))
 (segment (start 15.24 -32.385) (end 15.24 -38.1) (width 0.25) (layer "F.Cu") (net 30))
 (segment (start 14.08 -5.54) (end 12.35 -3.81) (width 0.25) (layer "F.Cu") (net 30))
 (segment (start 30.48 -74.93) (end 29.115 -73.565) (width 0.25) (layer "F.Cu") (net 52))
 (segment (start 29.115 -71.025) (end 25.4 -67.31) (width 0.25) (layer "F.Cu") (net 52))
 (segment (start 25.4 -67.31) (end 25.4 -63.5) (width 0.25) (layer "F.Cu") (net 52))
 (segment (start 29.115 -73.565) (end 29.115 -71.025) (width 0.25) (layer "F.Cu") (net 52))
 (segment (start 30.48 -72.39) (end 30.48 -70.485) (width 0.25) (layer "F.Cu") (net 51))
 (segment (start 27.94 -67.945) (end 27.94 -63.5) (width 0.25) (layer "F.Cu") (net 51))
 (segment (start 30.48 -70.485) (end 27.94 -67.945) (width 0.25) (layer "F.Cu") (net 51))
 (segment (start 31.75 -69.215) (end 30.48 -67.945) (width 0.25) (layer "F.Cu") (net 50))
 (segment (start 31.75 -73.66) (end 31.75 -69.215) (width 0.25) (layer "F.Cu") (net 50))
 (segment (start 33.02 -74.93) (end 31.75 -73.66) (width 0.25) (layer "F.Cu") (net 50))
 (segment (start 30.48 -67.945) (end 30.48 -63.5) (width 0.25) (layer "F.Cu") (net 50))
 (segment (start 33.02 -72.39) (end 33.02 -63.5) (width 0.25) (layer "F.Cu") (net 49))
 (segment (start 34.29 -73.66) (end 34.29 -68.58) (width 0.25) (layer "F.Cu") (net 48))
 (segment (start 35.56 -74.93) (end 34.29 -73.66) (width 0.25) (layer "F.Cu") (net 48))
 (segment (start 35.56 -67.31) (end 35.56 -63.5) (width 0.25) (layer "F.Cu") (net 48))
 (segment (start 34.29 -68.58) (end 35.56 -67.31) (width 0.25) (layer "F.Cu") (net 48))
 (segment (start 38.1 -66.675) (end 38.1 -63.5) (width 0.25) (layer "F.Cu") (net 47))
 (segment (start 35.56 -69.215) (end 38.1 -66.675) (width 0.25) (layer "F.Cu") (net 47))
 (segment (start 35.56 -72.39) (end 35.56 -69.215) (width 0.25) (layer "F.Cu") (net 47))
 (segment (start 36.83 -73.66) (end 36.83 -69.85) (width 0.25) (layer "F.Cu") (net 46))
 (segment (start 38.1 -74.93) (end 36.83 -73.66) (width 0.25) (layer "F.Cu") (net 46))
 (segment (start 40.64 -66.04) (end 40.64 -63.5) (width 0.25) (layer "F.Cu") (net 46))
 (segment (start 36.83 -69.85) (end 40.64 -66.04) (width 0.25) (layer "F.Cu") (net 46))
 (segment (start 38.1 -70.485) (end 43.18 -65.405) (width 0.25) (layer "F.Cu") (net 45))
 (segment (start 38.1 -72.39) (end 38.1 -70.485) (width 0.25) (layer "F.Cu") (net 45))
 (segment (start 43.18 -65.405) (end 43.18 -63.5) (width 0.25) (layer "F.Cu") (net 45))
 (segment (start 49.64 -22.97) (end 60.96 -34.29) (width 0.25) (layer "F.Cu") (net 5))
 (segment (start 54.61 -73.66) (end 54.61 -59.69) (width 0.25) (layer "F.Cu") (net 5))
 (segment (start 54.61 -59.69) (end 55.245 -59.055) (width 0.25) (layer "F.Cu") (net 5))
 (segment (start 60.96 -34.29) (end 60.96 -38.1) (width 0.25) (layer "F.Cu") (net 5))
 (segment (start 53.34 -74.93) (end 54.61 -73.66) (width 0.25) (layer "F.Cu") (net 5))
 (segment (start 49.64 -8.08) (end 49.64 -22.97) (width 0.25) (layer "F.Cu") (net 5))
 (segment (start 48.26 -74.93) (end 53.34 -74.93) (width 0.25) (layer "F.Cu") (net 5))
 (via (at 55.245 -59.055) (size 0.8) (drill 0.4) (layers "F.Cu" "B.Cu") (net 5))
 (segment (start 36.94 -5.54) (end 36.94 -6.875) (width 0.25) (layer "B.Cu") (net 5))
 (segment (start 55.245 -59.055) (end 60.96 -53.34) (width 0.25) (layer "B.Cu") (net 5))
 (segment (start 12.065 -59.055) (end 55.245 -59.055) (width 0.25) (layer "B.Cu") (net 5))
 (segment (start 10.16 -60.96) (end 12.065 -59.055) (width 0.25) (layer "B.Cu") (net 5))
 (segment (start 36.94 -6.875) (end 36.91 -6.905) (width 0.25) (layer "B.Cu") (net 5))
 (segment (start 14.255 -10.795) (end 26.605 -10.795) (width 0.25) (layer "B.Cu") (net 5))
 (segment (start 9.065 -8.08) (end 11.54 -8.08) (width 0.25) (layer "B.Cu") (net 5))
 (segment (start 48.465 -6.905) (end 49.64 -8.08) (width 0.25) (layer "B.Cu") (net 5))
 (segment (start 30.495 -6.905) (end 36.91 -6.905) (width 0.25) (layer "B.Cu") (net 5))
 (segment (start 10.16 -63.5) (end 10.16 -60.96) (width 0.25) (layer "B.Cu") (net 5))
 (segment (start 26.605 -10.795) (end 29.32 -8.08) (width 0.25) (layer "B.Cu") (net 5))
 (segment (start 60.96 -53.34) (end 60.96 -38.1) (width 0.25) (layer "B.Cu") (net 5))
 (segment (start 11.54 -8.08) (end 14.255 -10.795) (width 0.25) (layer "B.Cu") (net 5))
 (segment (start 29.32 -8.08) (end 30.495 -6.905) (width 0.25) (layer "B.Cu") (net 5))
 (segment (start 6.35 -10.795) (end 9.065 -8.08) (width 0.25) (layer "B.Cu") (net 5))
 (segment (start 6.35 -16.55) (end 6.35 -10.795) (width 0.25) (layer "B.Cu") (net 5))
 (segment (start 36.91 -6.905) (end 48.465 -6.905) (width 0.25) (layer "B.Cu") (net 5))
 (segment (start 50.8 -38.1) (end 50.8 -23.495) (width 0.25) (layer "B.Cu") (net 36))
 (segment (start 61.595 -12.7) (end 66.04 -12.7) (width 0.25) (layer "B.Cu") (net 36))
 (segment (start 50.8 -23.495) (end 61.595 -12.7) (width 0.25) (layer "B.Cu") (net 36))
 (segment (start 62.23 -15.24) (end 66.04 -15.24) (width 0.25) (layer "B.Cu") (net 35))
 (segment (start 53.34 -24.13) (end 62.23 -15.24) (width 0.25) (layer "B.Cu") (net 35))
 (segment (start 53.34 -38.1) (end 53.34 -24.13) (width 0.25) (layer "B.Cu") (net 35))
 (segment (start 55.88 -38.1) (end 55.88 -24.13) (width 0.25) (layer "B.Cu") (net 34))
 (segment (start 55.88 -24.13) (end 62.23 -17.78) (width 0.25) (layer "B.Cu") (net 34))
 (segment (start 62.23 -17.78) (end 66.04 -17.78) (width 0.25) (layer "B.Cu") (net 34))
 (segment (start 62.865 -20.32) (end 59.055 -24.13) (width 0.25) (layer "B.Cu") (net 33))
 (segment (start 59.055 -31.75) (end 62.865 -35.56) (width 0.25) (layer "B.Cu") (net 33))
 (segment (start 62.865 -35.56) (end 62.865 -53.975) (width 0.25) (layer "B.Cu") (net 33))
 (segment (start 59.055 -24.13) (end 59.055 -31.75) (width 0.25) (layer "B.Cu") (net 33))
 (segment (start 66.04 -20.32) (end 62.865 -20.32) (width 0.25) (layer "B.Cu") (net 33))
 (segment (start 62.865 -53.975) (end 55.88 -60.96) (width 0.25) (layer "B.Cu") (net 33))
 (segment (start 55.88 -60.96) (end 55.88 -63.5) (width 0.25) (layer "B.Cu") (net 33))
 (segment (start 60.325 -25.4) (end 62.865 -22.86) (width 0.25) (layer "B.Cu") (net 32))
 (segment (start 62.865 -22.86) (end 66.04 -22.86) (width 0.25) (layer "B.Cu") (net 32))
 (segment (start 60.325 -30.48) (end 60.325 -25.4) (width 0.25) (layer "B.Cu") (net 32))
 (segment (start 58.42 -61.595) (end 64.135 -55.88) (width 0.25) (layer "B.Cu") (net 32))
 (segment (start 64.135 -55.88) (end 64.135 -34.29) (width 0.25) (layer "B.Cu") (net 32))
 (segment (start 58.42 -63.5) (end 58.42 -61.595) (width 0.25) (layer "B.Cu") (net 32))
 (segment (start 64.135 -34.29) (end 60.325 -30.48) (width 0.25) (layer "B.Cu") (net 32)))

